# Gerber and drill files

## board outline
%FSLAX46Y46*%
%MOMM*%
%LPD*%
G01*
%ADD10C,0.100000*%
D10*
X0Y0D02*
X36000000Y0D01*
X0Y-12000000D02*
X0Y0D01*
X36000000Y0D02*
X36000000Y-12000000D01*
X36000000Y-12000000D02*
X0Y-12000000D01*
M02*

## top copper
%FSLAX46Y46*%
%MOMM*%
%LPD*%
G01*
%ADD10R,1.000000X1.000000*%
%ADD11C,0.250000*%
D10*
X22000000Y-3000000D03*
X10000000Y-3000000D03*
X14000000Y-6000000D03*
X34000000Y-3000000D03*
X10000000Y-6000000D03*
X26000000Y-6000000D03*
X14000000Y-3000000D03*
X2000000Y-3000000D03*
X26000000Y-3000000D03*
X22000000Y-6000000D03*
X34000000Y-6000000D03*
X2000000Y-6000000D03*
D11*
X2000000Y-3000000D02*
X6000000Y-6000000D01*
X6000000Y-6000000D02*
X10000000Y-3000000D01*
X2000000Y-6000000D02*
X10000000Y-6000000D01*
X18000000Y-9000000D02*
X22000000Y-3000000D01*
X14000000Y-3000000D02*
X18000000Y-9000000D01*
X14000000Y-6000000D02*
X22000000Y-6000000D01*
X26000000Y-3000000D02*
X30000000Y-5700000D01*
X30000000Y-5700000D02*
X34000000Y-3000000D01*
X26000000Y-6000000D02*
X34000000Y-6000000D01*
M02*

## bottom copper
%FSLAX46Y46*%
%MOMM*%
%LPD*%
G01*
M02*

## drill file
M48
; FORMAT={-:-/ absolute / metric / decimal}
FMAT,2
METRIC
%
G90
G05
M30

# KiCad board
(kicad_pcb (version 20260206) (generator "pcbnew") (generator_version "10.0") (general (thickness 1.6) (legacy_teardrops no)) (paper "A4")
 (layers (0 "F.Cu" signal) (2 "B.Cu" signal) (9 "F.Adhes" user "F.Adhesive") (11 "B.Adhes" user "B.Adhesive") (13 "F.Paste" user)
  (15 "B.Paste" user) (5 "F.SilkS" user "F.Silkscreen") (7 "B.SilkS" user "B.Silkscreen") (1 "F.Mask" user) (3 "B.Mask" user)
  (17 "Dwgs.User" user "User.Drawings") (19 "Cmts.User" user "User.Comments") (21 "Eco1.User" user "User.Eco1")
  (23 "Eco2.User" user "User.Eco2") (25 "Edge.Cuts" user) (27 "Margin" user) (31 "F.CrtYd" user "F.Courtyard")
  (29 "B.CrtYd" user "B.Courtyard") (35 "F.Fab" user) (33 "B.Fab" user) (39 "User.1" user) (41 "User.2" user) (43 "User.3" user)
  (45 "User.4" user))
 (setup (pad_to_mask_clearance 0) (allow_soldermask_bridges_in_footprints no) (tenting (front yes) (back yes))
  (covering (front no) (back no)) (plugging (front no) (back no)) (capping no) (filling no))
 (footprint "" (layer "F.Cu") (at 22 3)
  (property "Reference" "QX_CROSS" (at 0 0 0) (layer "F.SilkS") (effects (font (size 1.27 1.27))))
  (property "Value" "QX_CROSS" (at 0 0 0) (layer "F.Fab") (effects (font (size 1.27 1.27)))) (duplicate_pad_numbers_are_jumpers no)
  (pad "1" smd rect (at 0 0) (size 1 1) (layers "F.Cu" "F.Mask" "F.Paste") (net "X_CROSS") (thermal_bridge_angle 45)))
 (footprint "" (layer "F.Cu") (at 10 3)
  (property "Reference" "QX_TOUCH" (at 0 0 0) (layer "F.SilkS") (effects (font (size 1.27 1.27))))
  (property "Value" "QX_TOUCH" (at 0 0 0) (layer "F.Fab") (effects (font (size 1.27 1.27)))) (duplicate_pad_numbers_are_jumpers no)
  (pad "1" smd rect (at 0 0) (size 1 1) (layers "F.Cu" "F.Mask" "F.Paste") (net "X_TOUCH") (thermal_bridge_angle 45)))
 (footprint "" (layer "F.Cu") (at 14 6)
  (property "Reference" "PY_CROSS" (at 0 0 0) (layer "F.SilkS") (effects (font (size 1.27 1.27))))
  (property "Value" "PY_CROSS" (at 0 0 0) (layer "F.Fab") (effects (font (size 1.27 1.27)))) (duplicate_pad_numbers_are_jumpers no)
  (pad "1" smd rect (at 0 0) (size 1 1) (layers "F.Cu" "F.Mask" "F.Paste") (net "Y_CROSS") (thermal_bridge_angle 45)))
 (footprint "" (layer "F.Cu") (at 34 3)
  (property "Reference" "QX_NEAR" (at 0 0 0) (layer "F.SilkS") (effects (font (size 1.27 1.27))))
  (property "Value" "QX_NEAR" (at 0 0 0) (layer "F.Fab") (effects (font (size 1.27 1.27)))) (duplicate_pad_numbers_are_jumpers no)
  (pad "1" smd rect (at 0 0) (size 1 1) (layers "F.Cu" "F.Mask" "F.Paste") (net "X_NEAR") (thermal_bridge_angle 45)))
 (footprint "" (layer "F.Cu") (at 10 6)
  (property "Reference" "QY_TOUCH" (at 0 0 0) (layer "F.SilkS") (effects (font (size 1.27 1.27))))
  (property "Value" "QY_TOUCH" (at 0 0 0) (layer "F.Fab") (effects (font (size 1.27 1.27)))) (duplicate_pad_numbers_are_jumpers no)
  (pad "1" smd rect (at 0 0) (size 1 1) (layers "F.Cu" "F.Mask" "F.Paste") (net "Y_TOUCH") (thermal_bridge_angle 45)))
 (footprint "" (layer "F.Cu") (at 26 6)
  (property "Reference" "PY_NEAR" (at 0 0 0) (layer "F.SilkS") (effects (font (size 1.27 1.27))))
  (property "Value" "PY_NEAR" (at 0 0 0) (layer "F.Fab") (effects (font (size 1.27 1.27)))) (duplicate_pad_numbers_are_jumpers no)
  (pad "1" smd rect (at 0 0) (size 1 1) (layers "F.Cu" "F.Mask" "F.Paste") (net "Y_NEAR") (thermal_bridge_angle 45)))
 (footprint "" (layer "F.Cu") (at 14 3)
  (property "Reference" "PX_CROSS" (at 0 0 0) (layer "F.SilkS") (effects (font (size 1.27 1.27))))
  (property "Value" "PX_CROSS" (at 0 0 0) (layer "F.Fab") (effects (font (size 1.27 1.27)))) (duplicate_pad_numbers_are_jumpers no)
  (pad "1" smd rect (at 0 0) (size 1 1) (layers "F.Cu" "F.Mask" "F.Paste") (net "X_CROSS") (thermal_bridge_angle 45)))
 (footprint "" (layer "F.Cu") (at 2 3)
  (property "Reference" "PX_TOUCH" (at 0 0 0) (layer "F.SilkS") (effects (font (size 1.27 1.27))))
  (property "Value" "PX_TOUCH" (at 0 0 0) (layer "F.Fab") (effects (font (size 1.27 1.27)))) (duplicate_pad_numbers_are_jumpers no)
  (pad "1" smd rect (at 0 0) (size 1 1) (layers "F.Cu" "F.Mask" "F.Paste") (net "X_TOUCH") (thermal_bridge_angle 45)))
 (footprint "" (layer "F.Cu") (at 26 3)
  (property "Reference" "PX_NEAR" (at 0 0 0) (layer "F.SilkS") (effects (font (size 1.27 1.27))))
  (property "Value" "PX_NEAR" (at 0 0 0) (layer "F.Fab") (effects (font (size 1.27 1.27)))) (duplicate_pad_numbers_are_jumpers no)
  (pad "1" smd rect (at 0 0) (size 1 1) (layers "F.Cu" "F.Mask" "F.Paste") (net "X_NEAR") (thermal_bridge_angle 45)))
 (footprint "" (layer "F.Cu") (at 22 6)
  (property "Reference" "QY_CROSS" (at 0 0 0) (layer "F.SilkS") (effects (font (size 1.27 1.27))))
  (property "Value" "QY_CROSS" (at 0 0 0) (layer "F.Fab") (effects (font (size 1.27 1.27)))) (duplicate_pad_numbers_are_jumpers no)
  (pad "1" smd rect (at 0 0) (size 1 1) (layers "F.Cu" "F.Mask" "F.Paste") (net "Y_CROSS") (thermal_bridge_angle 45)))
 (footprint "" (layer "F.Cu") (at 34 6)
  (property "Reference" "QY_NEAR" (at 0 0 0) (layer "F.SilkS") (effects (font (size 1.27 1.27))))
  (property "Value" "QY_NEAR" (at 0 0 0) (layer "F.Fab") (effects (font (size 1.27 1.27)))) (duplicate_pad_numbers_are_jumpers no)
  (pad "1" smd rect (at 0 0) (size 1 1) (layers "F.Cu" "F.Mask" "F.Paste") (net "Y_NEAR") (thermal_bridge_angle 45)))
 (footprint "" (layer "F.Cu") (at 2 6)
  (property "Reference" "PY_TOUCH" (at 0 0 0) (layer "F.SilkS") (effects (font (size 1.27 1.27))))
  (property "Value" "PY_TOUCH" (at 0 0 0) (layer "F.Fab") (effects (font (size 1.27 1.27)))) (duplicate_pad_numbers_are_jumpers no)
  (pad "1" smd rect (at 0 0) (size 1 1) (layers "F.Cu" "F.Mask" "F.Paste") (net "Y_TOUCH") (thermal_bridge_angle 45)))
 (gr_line (start 0 0) (end 36 0) (stroke (width 0.1) (type default)) (layer "Edge.Cuts"))
 (gr_line (start 0 12) (end 0 0) (stroke (width 0.1) (type default)) (layer "Edge.Cuts"))
 (gr_line (start 36 0) (end 36 12) (stroke (width 0.1) (type default)) (layer "Edge.Cuts"))
 (gr_line (start 36 12) (end 0 12) (stroke (width 0.1) (type default)) (layer "Edge.Cuts"))
 (segment (start 2 3) (end 6 6) (width 0.25) (layer "F.Cu") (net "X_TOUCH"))
 (segment (start 6 6) (end 10 3) (width 0.25) (layer "F.Cu") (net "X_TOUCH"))
 (segment (start 2 6) (end 10 6) (width 0.25) (layer "F.Cu") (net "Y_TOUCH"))
 (segment (start 18 9) (end 22 3) (width 0.25) (layer "F.Cu") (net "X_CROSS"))
 (segment (start 14 3) (end 18 9) (width 0.25) (layer "F.Cu") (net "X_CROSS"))
 (segment (start 14 6) (end 22 6) (width 0.25) (layer "F.Cu") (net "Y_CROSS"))
 (segment (start 26 3) (end 30 5.7) (width 0.25) (layer "F.Cu") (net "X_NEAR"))
 (segment (start 30 5.7) (end 34 3) (width 0.25) (layer "F.Cu") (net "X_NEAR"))
 (segment (start 26 6) (end 34 6) (width 0.25) (layer "F.Cu") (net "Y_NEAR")))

